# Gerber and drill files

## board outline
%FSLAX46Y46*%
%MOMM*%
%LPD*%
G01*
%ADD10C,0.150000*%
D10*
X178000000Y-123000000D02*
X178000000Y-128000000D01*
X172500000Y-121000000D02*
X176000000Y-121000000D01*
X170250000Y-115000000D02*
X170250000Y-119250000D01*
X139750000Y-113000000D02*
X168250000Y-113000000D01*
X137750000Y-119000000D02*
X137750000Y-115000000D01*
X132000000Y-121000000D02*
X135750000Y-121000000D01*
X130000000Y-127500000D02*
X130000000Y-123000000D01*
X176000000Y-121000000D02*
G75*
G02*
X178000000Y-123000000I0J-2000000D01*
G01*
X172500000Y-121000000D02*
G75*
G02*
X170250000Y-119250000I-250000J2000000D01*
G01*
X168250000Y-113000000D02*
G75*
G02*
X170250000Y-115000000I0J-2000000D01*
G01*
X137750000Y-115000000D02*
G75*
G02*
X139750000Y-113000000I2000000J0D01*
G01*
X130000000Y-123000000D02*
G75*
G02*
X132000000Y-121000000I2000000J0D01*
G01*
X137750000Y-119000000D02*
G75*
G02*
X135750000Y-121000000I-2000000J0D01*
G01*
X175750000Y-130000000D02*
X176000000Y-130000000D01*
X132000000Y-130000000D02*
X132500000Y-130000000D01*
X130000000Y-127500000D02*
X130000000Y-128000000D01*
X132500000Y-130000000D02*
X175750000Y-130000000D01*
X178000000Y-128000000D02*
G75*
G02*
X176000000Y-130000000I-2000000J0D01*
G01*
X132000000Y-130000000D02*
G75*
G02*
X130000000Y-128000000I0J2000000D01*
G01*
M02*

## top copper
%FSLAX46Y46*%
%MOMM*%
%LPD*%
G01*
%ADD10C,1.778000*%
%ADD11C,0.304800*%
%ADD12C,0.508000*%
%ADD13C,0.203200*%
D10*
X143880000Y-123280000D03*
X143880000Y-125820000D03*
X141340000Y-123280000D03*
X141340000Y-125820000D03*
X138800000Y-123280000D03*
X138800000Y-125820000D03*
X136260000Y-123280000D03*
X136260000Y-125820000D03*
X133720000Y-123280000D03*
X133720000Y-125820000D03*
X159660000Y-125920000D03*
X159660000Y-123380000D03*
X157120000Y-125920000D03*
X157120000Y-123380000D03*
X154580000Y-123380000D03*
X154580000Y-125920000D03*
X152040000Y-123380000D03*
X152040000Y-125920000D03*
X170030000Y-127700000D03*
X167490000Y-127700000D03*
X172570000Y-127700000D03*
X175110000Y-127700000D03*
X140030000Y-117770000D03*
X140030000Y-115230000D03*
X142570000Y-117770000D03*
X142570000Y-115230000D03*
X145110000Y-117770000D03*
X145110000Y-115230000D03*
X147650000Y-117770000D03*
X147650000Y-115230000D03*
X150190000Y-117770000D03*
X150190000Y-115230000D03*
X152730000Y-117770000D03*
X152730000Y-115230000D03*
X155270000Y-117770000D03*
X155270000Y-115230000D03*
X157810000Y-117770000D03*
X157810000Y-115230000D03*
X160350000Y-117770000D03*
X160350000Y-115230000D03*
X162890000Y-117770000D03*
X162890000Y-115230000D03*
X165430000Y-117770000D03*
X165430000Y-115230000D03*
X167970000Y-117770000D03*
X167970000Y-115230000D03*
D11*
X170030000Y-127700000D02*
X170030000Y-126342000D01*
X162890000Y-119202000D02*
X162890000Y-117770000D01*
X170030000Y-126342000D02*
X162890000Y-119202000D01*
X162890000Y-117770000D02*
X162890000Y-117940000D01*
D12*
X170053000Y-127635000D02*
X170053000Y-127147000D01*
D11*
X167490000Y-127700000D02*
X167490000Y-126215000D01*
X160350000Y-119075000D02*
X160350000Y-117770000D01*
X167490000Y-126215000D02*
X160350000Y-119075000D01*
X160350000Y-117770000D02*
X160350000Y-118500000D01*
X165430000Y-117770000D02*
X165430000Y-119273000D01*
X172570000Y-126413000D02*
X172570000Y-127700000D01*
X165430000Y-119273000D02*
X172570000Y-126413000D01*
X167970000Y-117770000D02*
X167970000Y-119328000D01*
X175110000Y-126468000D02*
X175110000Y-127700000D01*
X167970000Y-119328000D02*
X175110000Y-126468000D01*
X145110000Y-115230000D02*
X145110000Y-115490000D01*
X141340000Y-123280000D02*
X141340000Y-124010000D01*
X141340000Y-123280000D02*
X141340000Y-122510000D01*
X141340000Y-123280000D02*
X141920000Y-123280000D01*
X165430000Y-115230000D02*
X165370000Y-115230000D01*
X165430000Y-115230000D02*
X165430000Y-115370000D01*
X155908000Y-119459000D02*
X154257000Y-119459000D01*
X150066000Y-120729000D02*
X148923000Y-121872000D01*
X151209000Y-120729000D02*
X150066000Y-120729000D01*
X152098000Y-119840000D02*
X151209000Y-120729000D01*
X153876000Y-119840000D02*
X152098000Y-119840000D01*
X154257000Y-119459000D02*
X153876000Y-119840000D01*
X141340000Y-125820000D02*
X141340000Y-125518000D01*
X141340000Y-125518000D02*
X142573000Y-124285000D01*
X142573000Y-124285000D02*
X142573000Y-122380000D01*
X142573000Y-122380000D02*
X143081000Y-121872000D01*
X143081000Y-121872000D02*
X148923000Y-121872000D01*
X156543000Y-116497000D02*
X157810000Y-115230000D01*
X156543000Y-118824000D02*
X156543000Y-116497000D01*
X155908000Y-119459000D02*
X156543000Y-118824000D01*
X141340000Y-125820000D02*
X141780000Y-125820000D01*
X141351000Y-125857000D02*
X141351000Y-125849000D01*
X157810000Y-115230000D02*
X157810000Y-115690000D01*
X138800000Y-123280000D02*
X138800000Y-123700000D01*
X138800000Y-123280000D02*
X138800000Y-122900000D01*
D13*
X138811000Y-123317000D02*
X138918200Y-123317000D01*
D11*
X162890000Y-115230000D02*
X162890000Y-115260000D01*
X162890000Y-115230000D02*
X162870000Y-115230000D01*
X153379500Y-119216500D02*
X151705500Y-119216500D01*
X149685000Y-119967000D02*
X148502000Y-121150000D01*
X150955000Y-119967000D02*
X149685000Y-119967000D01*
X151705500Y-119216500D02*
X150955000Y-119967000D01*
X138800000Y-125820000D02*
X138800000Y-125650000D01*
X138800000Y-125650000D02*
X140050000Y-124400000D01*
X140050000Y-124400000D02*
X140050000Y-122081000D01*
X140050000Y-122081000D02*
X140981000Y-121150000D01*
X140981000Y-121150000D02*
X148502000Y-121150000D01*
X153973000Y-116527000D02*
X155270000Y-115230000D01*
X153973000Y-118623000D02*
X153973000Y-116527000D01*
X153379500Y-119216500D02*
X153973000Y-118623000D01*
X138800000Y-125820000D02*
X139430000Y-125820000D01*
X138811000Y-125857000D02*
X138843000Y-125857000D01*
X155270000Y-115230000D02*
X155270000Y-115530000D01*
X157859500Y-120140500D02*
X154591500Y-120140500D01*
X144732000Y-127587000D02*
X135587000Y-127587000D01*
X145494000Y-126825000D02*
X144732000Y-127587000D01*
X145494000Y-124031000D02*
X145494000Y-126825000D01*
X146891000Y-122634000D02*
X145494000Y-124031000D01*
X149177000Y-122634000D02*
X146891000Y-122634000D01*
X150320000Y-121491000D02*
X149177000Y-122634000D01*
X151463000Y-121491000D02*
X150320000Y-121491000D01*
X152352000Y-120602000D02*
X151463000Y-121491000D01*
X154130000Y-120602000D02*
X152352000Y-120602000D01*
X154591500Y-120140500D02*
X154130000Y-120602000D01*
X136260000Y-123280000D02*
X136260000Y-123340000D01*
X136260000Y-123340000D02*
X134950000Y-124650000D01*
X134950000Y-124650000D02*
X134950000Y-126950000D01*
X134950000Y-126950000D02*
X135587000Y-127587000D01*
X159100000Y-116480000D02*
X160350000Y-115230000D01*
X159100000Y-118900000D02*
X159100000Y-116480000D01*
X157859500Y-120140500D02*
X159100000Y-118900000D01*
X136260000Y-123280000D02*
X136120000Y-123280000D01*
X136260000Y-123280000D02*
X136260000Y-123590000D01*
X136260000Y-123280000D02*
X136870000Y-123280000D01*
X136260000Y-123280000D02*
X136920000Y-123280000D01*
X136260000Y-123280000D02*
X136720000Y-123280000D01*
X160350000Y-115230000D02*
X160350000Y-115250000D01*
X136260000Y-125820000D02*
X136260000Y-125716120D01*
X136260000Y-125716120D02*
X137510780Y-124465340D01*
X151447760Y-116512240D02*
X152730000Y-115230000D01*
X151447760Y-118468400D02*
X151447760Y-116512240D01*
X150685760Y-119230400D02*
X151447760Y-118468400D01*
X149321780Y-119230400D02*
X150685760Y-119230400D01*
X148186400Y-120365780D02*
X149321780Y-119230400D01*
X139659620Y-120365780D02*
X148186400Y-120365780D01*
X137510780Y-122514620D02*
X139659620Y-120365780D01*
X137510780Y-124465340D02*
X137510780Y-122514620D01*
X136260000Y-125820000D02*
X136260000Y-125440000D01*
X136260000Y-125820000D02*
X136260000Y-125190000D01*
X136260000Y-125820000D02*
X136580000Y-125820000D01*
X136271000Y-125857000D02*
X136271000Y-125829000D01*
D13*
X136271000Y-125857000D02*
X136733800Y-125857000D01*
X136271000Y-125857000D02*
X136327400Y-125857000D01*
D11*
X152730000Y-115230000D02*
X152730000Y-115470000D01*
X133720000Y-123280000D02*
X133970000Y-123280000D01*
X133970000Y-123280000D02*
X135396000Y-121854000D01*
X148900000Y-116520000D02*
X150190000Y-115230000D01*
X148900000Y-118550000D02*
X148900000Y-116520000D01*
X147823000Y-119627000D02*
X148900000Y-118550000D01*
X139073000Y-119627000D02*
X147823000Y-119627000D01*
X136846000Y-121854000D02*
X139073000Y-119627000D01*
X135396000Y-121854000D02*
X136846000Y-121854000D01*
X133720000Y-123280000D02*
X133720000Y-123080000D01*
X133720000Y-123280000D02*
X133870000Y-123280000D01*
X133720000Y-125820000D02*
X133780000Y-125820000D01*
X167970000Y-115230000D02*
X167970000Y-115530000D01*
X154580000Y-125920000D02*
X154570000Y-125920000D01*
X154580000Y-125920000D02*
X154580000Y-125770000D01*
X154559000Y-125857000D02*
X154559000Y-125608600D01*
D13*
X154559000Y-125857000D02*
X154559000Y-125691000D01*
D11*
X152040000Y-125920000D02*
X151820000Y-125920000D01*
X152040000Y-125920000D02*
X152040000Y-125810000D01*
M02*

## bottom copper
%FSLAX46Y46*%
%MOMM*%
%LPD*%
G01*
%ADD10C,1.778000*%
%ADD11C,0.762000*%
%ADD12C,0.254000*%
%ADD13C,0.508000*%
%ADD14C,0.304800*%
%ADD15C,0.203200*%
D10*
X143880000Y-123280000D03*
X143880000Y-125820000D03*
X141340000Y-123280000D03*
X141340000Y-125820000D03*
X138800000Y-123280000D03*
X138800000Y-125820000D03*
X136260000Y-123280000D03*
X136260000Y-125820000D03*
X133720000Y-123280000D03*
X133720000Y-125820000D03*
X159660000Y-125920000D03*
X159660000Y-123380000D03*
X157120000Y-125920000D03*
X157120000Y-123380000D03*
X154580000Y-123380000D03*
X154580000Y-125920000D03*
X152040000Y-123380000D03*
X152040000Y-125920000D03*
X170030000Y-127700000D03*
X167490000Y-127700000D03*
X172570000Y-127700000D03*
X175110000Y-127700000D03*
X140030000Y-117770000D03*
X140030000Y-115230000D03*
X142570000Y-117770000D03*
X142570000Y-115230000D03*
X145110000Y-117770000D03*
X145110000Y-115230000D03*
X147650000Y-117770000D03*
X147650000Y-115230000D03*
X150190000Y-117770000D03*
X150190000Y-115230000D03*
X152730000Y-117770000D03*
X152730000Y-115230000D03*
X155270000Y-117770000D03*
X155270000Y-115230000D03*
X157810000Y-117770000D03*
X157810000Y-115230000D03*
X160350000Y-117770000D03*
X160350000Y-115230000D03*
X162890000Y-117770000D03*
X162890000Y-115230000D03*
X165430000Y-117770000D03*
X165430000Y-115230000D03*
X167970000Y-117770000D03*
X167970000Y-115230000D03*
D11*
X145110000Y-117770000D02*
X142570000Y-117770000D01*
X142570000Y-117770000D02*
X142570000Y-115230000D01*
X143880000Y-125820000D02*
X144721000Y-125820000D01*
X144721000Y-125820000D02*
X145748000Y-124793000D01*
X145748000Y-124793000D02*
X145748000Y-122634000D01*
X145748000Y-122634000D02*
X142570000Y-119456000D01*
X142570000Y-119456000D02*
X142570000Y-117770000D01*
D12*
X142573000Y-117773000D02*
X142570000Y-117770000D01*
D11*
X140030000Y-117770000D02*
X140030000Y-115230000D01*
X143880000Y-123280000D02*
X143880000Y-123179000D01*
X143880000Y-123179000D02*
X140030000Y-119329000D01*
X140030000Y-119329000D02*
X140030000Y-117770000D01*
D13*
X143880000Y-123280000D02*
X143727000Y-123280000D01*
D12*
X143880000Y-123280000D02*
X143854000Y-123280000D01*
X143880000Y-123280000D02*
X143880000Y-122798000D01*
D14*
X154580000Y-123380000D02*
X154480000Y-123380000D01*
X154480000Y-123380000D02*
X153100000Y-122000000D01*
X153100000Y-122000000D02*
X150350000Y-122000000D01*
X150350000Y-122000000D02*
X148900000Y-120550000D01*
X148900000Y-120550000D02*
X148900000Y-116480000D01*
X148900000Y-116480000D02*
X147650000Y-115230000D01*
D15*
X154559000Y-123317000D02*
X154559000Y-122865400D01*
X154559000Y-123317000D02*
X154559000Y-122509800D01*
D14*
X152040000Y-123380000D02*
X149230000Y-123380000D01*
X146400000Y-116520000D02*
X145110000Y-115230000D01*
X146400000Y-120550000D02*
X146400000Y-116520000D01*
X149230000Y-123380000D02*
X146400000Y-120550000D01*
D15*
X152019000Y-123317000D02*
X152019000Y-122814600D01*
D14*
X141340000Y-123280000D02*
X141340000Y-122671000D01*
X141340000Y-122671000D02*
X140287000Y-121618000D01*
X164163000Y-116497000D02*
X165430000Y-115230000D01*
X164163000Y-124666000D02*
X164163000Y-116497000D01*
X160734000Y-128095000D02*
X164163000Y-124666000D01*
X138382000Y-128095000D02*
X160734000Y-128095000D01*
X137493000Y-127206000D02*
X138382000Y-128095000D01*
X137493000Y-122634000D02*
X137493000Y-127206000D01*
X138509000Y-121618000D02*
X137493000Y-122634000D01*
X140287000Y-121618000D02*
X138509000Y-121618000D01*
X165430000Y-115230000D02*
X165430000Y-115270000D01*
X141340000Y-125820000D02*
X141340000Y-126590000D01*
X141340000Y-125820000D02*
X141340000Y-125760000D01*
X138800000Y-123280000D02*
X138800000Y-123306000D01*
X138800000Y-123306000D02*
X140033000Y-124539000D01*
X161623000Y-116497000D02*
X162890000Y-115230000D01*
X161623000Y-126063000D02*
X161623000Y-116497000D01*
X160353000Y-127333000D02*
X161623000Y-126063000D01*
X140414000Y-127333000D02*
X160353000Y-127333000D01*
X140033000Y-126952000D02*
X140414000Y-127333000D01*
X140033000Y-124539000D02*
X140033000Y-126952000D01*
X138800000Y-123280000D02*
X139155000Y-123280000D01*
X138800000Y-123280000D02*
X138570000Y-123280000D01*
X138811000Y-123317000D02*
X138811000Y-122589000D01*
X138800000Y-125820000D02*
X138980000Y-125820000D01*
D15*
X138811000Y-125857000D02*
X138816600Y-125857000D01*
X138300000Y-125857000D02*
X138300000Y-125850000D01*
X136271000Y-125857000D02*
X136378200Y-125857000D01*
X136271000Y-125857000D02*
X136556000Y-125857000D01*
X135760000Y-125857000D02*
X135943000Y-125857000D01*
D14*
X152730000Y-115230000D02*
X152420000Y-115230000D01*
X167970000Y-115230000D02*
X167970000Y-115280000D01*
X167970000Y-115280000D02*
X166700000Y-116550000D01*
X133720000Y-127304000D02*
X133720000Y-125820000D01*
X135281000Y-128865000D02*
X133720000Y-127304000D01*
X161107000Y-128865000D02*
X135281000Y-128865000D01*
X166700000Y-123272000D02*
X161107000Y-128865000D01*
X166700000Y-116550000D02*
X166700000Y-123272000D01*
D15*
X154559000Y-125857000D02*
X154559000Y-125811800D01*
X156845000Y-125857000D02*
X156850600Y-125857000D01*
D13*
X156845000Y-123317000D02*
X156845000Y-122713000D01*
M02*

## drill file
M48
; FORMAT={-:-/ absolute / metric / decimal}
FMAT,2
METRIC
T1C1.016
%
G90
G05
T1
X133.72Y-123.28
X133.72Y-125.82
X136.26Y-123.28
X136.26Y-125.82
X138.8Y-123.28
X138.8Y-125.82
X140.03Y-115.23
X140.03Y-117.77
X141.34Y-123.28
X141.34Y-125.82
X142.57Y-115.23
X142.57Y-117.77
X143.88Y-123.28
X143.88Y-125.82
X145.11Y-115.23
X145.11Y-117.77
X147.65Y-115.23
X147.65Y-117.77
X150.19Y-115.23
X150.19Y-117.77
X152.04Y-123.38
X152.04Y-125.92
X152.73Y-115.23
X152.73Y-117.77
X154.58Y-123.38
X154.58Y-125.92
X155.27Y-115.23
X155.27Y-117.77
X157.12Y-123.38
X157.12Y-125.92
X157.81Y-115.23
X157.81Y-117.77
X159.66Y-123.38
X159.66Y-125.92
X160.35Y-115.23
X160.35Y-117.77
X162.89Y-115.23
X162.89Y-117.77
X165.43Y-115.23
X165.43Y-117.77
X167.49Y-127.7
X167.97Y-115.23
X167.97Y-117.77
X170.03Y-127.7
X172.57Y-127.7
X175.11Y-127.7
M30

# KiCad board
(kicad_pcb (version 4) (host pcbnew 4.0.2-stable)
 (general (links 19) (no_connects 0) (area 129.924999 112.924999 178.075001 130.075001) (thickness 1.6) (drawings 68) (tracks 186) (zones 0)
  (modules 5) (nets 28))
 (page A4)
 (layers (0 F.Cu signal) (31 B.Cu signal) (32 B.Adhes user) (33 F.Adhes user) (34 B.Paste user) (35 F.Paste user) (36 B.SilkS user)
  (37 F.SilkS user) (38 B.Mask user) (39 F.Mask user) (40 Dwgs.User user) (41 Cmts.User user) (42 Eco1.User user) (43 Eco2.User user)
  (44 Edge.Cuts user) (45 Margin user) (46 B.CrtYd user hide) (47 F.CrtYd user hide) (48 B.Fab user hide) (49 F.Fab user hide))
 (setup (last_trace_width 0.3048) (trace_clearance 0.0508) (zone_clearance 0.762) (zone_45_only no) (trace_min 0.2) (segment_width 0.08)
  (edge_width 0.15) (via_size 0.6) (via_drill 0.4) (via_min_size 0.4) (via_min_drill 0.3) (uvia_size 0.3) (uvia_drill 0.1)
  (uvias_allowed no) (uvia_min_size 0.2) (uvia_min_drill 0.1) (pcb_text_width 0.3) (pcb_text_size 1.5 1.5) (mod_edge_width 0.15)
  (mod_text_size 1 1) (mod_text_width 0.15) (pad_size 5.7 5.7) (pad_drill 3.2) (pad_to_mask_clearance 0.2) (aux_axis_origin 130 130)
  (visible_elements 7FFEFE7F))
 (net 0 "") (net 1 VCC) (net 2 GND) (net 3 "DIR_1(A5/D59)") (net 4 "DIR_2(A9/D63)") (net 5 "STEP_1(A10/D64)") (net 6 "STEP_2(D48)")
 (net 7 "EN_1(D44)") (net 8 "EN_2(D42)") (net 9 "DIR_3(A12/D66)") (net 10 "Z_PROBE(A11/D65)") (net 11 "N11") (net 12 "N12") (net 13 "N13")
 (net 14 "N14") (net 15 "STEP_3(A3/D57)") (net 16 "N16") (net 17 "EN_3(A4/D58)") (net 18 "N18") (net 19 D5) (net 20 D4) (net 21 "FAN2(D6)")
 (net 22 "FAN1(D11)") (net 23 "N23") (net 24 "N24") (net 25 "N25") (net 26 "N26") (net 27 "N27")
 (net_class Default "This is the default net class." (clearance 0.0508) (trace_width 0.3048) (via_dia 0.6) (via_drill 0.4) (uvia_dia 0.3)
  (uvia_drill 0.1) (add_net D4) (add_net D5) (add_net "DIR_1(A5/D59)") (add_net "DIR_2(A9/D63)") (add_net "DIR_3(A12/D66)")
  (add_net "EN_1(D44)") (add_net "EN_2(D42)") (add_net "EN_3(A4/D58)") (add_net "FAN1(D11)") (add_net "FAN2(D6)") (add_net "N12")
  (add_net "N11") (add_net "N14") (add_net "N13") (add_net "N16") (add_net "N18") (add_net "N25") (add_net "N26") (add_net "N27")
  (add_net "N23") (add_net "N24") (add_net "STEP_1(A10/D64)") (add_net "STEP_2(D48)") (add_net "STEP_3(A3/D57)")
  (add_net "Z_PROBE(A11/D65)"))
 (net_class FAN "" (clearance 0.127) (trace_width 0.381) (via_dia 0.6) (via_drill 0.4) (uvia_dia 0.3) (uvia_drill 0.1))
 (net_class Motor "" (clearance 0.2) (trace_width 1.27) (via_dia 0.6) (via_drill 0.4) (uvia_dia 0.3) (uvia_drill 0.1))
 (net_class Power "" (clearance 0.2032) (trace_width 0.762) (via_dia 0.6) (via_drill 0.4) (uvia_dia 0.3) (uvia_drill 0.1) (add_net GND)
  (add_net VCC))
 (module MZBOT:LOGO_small (layer F.Cu) (at 167.66058 124.78538)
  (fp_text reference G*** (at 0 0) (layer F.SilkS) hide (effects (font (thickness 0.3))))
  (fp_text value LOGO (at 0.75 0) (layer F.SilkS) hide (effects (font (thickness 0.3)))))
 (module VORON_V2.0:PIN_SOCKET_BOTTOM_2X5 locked (layer F.Cu) (at 138.8 124.55 180)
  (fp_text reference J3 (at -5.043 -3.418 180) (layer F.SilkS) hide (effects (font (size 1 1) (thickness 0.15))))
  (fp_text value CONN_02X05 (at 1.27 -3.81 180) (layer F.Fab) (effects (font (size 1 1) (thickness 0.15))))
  (pad 1 thru_hole circle (at -5.08 1.27 180) (size 1.778 1.778) (drill 1.016) (layers *.Cu *.Mask F.SilkS) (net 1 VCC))
  (pad 2 thru_hole circle (at -5.08 -1.27 180) (size 1.778 1.778) (drill 1.016) (layers *.Cu *.Mask F.SilkS) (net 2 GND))
  (pad 3 thru_hole circle (at -2.54 1.27 180) (size 1.778 1.778) (drill 1.016) (layers *.Cu *.Mask F.SilkS) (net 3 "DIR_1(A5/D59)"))
  (pad 4 thru_hole circle (at -2.54 -1.27 180) (size 1.778 1.778) (drill 1.016) (layers *.Cu *.Mask F.SilkS) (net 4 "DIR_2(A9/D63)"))
  (pad 5 thru_hole circle (at 0 1.27 180) (size 1.778 1.778) (drill 1.016) (layers *.Cu *.Mask F.SilkS) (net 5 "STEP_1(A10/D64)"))
  (pad 6 thru_hole circle (at 0 -1.27 180) (size 1.778 1.778) (drill 1.016) (layers *.Cu *.Mask F.SilkS) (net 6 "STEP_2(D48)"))
  (pad 7 thru_hole circle (at 2.54 1.27 180) (size 1.778 1.778) (drill 1.016) (layers *.Cu *.Mask F.SilkS) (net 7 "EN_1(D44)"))
  (pad 8 thru_hole circle (at 2.54 -1.27 180) (size 1.778 1.778) (drill 1.016) (layers *.Cu *.Mask F.SilkS) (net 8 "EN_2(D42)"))
  (pad 9 thru_hole circle (at 5.08 1.27 180) (size 1.778 1.778) (drill 1.016) (layers *.Cu *.Mask F.SilkS) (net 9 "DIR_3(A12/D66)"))
  (pad 10 thru_hole circle (at 5.08 -1.27 180) (size 1.778 1.778) (drill 1.016) (layers *.Cu *.Mask F.SilkS) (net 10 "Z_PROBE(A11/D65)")))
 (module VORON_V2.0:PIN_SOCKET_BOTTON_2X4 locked (layer F.Cu) (at 155.85 124.65 180)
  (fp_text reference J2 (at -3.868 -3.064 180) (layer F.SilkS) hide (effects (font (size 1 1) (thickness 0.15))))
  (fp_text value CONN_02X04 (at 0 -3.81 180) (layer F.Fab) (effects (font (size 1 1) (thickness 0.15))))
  (pad 2 thru_hole circle (at -3.81 -1.27 180) (size 1.778 1.778) (drill 1.016) (layers *.Cu *.Mask F.SilkS) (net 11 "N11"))
  (pad 1 thru_hole circle (at -3.81 1.27 180) (size 1.778 1.778) (drill 1.016) (layers *.Cu *.Mask F.SilkS) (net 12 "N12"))
  (pad 4 thru_hole circle (at -1.27 -1.27 180) (size 1.778 1.778) (drill 1.016) (layers *.Cu *.Mask F.SilkS) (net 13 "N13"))
  (pad 3 thru_hole circle (at -1.27 1.27 180) (size 1.778 1.778) (drill 1.016) (layers *.Cu *.Mask F.SilkS) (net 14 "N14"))
  (pad 5 thru_hole circle (at 1.27 1.27 180) (size 1.778 1.778) (drill 1.016) (layers *.Cu *.Mask F.SilkS) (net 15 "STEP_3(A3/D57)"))
  (pad 6 thru_hole circle (at 1.27 -1.27 180) (size 1.778 1.778) (drill 1.016) (layers *.Cu *.Mask F.SilkS) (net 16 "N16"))
  (pad 7 thru_hole circle (at 3.81 1.27 180) (size 1.778 1.778) (drill 1.016) (layers *.Cu *.Mask F.SilkS) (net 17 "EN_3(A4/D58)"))
  (pad 8 thru_hole circle (at 3.81 -1.27 180) (size 1.778 1.778) (drill 1.016) (layers *.Cu *.Mask F.SilkS) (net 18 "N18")))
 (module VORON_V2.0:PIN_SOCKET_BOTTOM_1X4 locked (layer F.Cu) (at 171.3 127.7)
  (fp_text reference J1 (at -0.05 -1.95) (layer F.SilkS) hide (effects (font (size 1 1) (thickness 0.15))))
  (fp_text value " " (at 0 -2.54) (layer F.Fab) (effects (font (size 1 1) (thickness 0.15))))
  (pad 2 thru_hole circle (at -1.27 0) (size 1.778 1.778) (drill 1.016) (layers *.Cu *.Mask F.SilkS) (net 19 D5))
  (pad 1 thru_hole circle (at -3.81 0) (size 1.778 1.778) (drill 1.016) (layers *.Cu *.Mask F.SilkS) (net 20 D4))
  (pad 3 thru_hole circle (at 1.27 0) (size 1.778 1.778) (drill 1.016) (layers *.Cu *.Mask F.SilkS) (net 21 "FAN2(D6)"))
  (pad 4 thru_hole circle (at 3.81 0) (size 1.778 1.778) (drill 1.016) (layers *.Cu *.Mask F.SilkS) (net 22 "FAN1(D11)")))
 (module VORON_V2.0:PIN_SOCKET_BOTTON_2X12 (layer F.Cu) (at 154 116.5)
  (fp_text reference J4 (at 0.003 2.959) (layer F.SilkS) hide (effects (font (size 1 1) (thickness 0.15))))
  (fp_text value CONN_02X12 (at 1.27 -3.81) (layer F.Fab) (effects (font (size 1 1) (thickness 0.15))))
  (pad 1 thru_hole circle (at -13.97 1.27) (size 1.778 1.778) (drill 1.016) (layers *.Cu *.Mask F.SilkS) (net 1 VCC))
  (pad 2 thru_hole circle (at -13.97 -1.27) (size 1.778 1.778) (drill 1.016) (layers *.Cu *.Mask F.SilkS) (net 1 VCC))
  (pad 3 thru_hole circle (at -11.43 1.27) (size 1.778 1.778) (drill 1.016) (layers *.Cu *.Mask F.SilkS) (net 2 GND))
  (pad 4 thru_hole circle (at -11.43 -1.27) (size 1.778 1.778) (drill 1.016) (layers *.Cu *.Mask F.SilkS) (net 2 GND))
  (pad 5 thru_hole circle (at -8.89 1.27) (size 1.778 1.778) (drill 1.016) (layers *.Cu *.Mask F.SilkS) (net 2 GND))
  (pad 6 thru_hole circle (at -8.89 -1.27) (size 1.778 1.778) (drill 1.016) (layers *.Cu *.Mask F.SilkS) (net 17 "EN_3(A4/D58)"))
  (pad 7 thru_hole circle (at -6.35 1.27) (size 1.778 1.778) (drill 1.016) (layers *.Cu *.Mask F.SilkS) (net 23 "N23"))
  (pad 8 thru_hole circle (at -6.35 -1.27) (size 1.778 1.778) (drill 1.016) (layers *.Cu *.Mask F.SilkS) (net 15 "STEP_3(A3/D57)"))
  (pad 9 thru_hole circle (at -3.81 1.27) (size 1.778 1.778) (drill 1.016) (layers *.Cu *.Mask F.SilkS) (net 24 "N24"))
  (pad 10 thru_hole circle (at -3.81 -1.27) (size 1.778 1.778) (drill 1.016) (layers *.Cu *.Mask F.SilkS) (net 9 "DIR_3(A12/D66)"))
  (pad 11 thru_hole circle (at -1.27 1.27) (size 1.778 1.778) (drill 1.016) (layers *.Cu *.Mask F.SilkS) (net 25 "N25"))
  (pad 12 thru_hole circle (at -1.27 -1.27) (size 1.778 1.778) (drill 1.016) (layers *.Cu *.Mask F.SilkS) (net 8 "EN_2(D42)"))
  (pad 13 thru_hole circle (at 1.27 1.27) (size 1.778 1.778) (drill 1.016) (layers *.Cu *.Mask F.SilkS) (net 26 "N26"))
  (pad 14 thru_hole circle (at 1.27 -1.27) (size 1.778 1.778) (drill 1.016) (layers *.Cu *.Mask F.SilkS) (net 6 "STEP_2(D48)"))
  (pad 15 thru_hole circle (at 3.81 1.27) (size 1.778 1.778) (drill 1.016) (layers *.Cu *.Mask F.SilkS) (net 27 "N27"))
  (pad 16 thru_hole circle (at 3.81 -1.27) (size 1.778 1.778) (drill 1.016) (layers *.Cu *.Mask F.SilkS) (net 4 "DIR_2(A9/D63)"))
  (pad 17 thru_hole circle (at 6.35 1.27) (size 1.778 1.778) (drill 1.016) (layers *.Cu *.Mask F.SilkS) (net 20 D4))
  (pad 18 thru_hole circle (at 6.35 -1.27) (size 1.778 1.778) (drill 1.016) (layers *.Cu *.Mask F.SilkS) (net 7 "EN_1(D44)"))
  (pad 19 thru_hole circle (at 8.89 1.27) (size 1.778 1.778) (drill 1.016) (layers *.Cu *.Mask F.SilkS) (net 19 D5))
  (pad 20 thru_hole circle (at 8.89 -1.27) (size 1.778 1.778) (drill 1.016) (layers *.Cu *.Mask F.SilkS) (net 5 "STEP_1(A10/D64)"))
  (pad 21 thru_hole circle (at 11.43 1.27) (size 1.778 1.778) (drill 1.016) (layers *.Cu *.Mask F.SilkS) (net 21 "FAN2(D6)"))
  (pad 22 thru_hole circle (at 11.43 -1.27) (size 1.778 1.778) (drill 1.016) (layers *.Cu *.Mask F.SilkS) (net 3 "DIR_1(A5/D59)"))
  (pad 23 thru_hole circle (at 13.97 1.27) (size 1.778 1.778) (drill 1.016) (layers *.Cu *.Mask F.SilkS) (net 22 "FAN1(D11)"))
  (pad 24 thru_hole circle (at 13.97 -1.27) (size 1.778 1.778) (drill 1.016) (layers *.Cu *.Mask F.SilkS) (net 10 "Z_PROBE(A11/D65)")))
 (gr_line (start 178 123) (end 178 128) (angle 90) (layer Edge.Cuts) (width 0.15))
 (gr_line (start 172.5 121) (end 176 121) (angle 90) (layer Edge.Cuts) (width 0.15))
 (gr_line (start 170.25 115) (end 170.25 119.25) (angle 90) (layer Edge.Cuts) (width 0.15))
 (gr_line (start 139.75 113) (end 168.25 113) (angle 90) (layer Edge.Cuts) (width 0.15))
 (gr_line (start 137.75 119) (end 137.75 115) (angle 90) (layer Edge.Cuts) (width 0.15))
 (gr_line (start 132 121) (end 135.75 121) (angle 90) (layer Edge.Cuts) (width 0.15))
 (gr_line (start 130 127.5) (end 130 123) (angle 90) (layer Edge.Cuts) (width 0.15))
 (gr_arc (start 176 123) (end 176 121) (angle 90) (layer Edge.Cuts) (width 0.15))
 (gr_arc (start 172.25 119) (end 172.5 121) (angle 90) (layer Edge.Cuts) (width 0.15))
 (gr_arc (start 168.25 115) (end 168.25 113) (angle 90) (layer Edge.Cuts) (width 0.15))
 (gr_arc (start 139.75 115) (end 137.75 115) (angle 90) (layer Edge.Cuts) (width 0.15))
 (gr_arc (start 132 123) (end 130 123) (angle 90) (layer Edge.Cuts) (width 0.15))
 (gr_arc (start 135.75 119) (end 137.75 119) (angle 90) (layer Edge.Cuts) (width 0.15))
 (gr_line (start 175.75 130) (end 176 130) (angle 90) (layer Edge.Cuts) (width 0.15))
 (gr_line (start 132 130) (end 132.5 130) (angle 90) (layer Edge.Cuts) (width 0.15))
 (gr_line (start 130 127.5) (end 130 128) (angle 90) (layer Edge.Cuts) (width 0.15))
 (gr_line (start 132.5 130) (end 175.75 130) (angle 90) (layer Edge.Cuts) (width 0.15))
 (gr_arc (start 176 128) (end 178 128) (angle 90) (layer Edge.Cuts) (width 0.15))
 (gr_arc (start 132 128) (end 132 130) (angle 90) (layer Edge.Cuts) (width 0.15))
 (segment (start 145.11 117.77) (end 142.57 117.77) (width 0.762) (layer B.Cu) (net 2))
 (segment (start 142.57 117.77) (end 142.57 115.23) (width 0.762) (layer B.Cu) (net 2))
 (segment (start 143.88 125.82) (end 144.721 125.82) (width 0.762) (layer B.Cu) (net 2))
 (segment (start 144.721 125.82) (end 145.748 124.793) (width 0.762) (layer B.Cu) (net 2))
 (segment (start 145.748 124.793) (end 145.748 122.634) (width 0.762) (layer B.Cu) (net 2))
 (segment (start 145.748 122.634) (end 142.57 119.456) (width 0.762) (layer B.Cu) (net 2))
 (segment (start 142.57 119.456) (end 142.57 117.77) (width 0.762) (layer B.Cu) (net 2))
 (segment (start 142.573 117.773) (end 142.57 117.77) (width 0.254) (layer B.Cu) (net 2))
 (segment (start 140.03 117.77) (end 140.03 115.23) (width 0.762) (layer B.Cu) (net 1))
 (segment (start 143.88 123.28) (end 143.88 123.179) (width 0.762) (layer B.Cu) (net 1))
 (segment (start 143.88 123.179) (end 140.03 119.329) (width 0.762) (layer B.Cu) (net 1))
 (segment (start 140.03 119.329) (end 140.03 117.77) (width 0.762) (layer B.Cu) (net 1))
 (segment (start 143.88 123.28) (end 143.727 123.28) (width 0.508) (layer B.Cu) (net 1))
 (segment (start 143.88 123.28) (end 143.854 123.28) (width 0.254) (layer B.Cu) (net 1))
 (segment (start 143.88 123.28) (end 143.88 122.798) (width 0.254) (layer B.Cu) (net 1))
 (segment (start 170.03 127.7) (end 170.03 126.342) (width 0.3048) (layer F.Cu) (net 19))
 (segment (start 162.89 119.202) (end 162.89 117.77) (width 0.3048) (layer F.Cu) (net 19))
 (segment (start 170.03 126.342) (end 162.89 119.202) (width 0.3048) (layer F.Cu) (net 19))
 (segment (start 162.89 117.77) (end 162.89 117.94) (width 0.3048) (layer F.Cu) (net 19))
 (segment (start 170.053 127.635) (end 170.053 127.147) (width 0.508) (layer F.Cu) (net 19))
 (segment (start 167.49 127.7) (end 167.49 126.215) (width 0.3048) (layer F.Cu) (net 20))
 (segment (start 160.35 119.075) (end 160.35 117.77) (width 0.3048) (layer F.Cu) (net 20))
 (segment (start 167.49 126.215) (end 160.35 119.075) (width 0.3048) (layer F.Cu) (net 20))
 (segment (start 160.35 117.77) (end 160.35 118.5) (width 0.3048) (layer F.Cu) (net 20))
 (segment (start 165.43 117.77) (end 165.43 119.273) (width 0.3048) (layer F.Cu) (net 21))
 (segment (start 172.57 126.413) (end 172.57 127.7) (width 0.3048) (layer F.Cu) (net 21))
 (segment (start 165.43 119.273) (end 172.57 126.413) (width 0.3048) (layer F.Cu) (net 21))
 (segment (start 167.97 117.77) (end 167.97 119.328) (width 0.3048) (layer F.Cu) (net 22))
 (segment (start 175.11 126.468) (end 175.11 127.7) (width 0.3048) (layer F.Cu) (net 22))
 (segment (start 167.97 119.328) (end 175.11 126.468) (width 0.3048) (layer F.Cu) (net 22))
 (segment (start 154.58 123.38) (end 154.48 123.38) (width 0.3048) (layer B.Cu) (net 15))
 (segment (start 154.48 123.38) (end 153.1 122) (width 0.3048) (layer B.Cu) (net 15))
 (segment (start 153.1 122) (end 150.35 122) (width 0.3048) (layer B.Cu) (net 15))
 (segment (start 150.35 122) (end 148.9 120.55) (width 0.3048) (layer B.Cu) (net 15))
 (segment (start 148.9 120.55) (end 148.9 116.48) (width 0.3048) (layer B.Cu) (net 15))
 (segment (start 148.9 116.48) (end 147.65 115.23) (width 0.3048) (layer B.Cu) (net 15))
 (segment (start 154.559 123.317) (end 154.559 122.8654) (width 0.2032) (layer B.Cu) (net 15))
 (segment (start 154.559 123.317) (end 154.559 122.5098) (width 0.2032) (layer B.Cu) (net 15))
 (segment (start 152.04 123.38) (end 149.23 123.38) (width 0.3048) (layer B.Cu) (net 17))
 (segment (start 146.4 116.52) (end 145.11 115.23) (width 0.3048) (layer B.Cu) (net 17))
 (segment (start 146.4 120.55) (end 146.4 116.52) (width 0.3048) (layer B.Cu) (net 17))
 (segment (start 149.23 123.38) (end 146.4 120.55) (width 0.3048) (layer B.Cu) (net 17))
 (segment (start 152.019 123.317) (end 152.019 122.8146) (width 0.2032) (layer B.Cu) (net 17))
 (segment (start 145.11 115.23) (end 145.11 115.49) (width 0.3048) (layer F.Cu) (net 17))
 (segment (start 141.34 123.28) (end 141.34 122.671) (width 0.3048) (layer B.Cu) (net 3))
 (segment (start 141.34 122.671) (end 140.287 121.618) (width 0.3048) (layer B.Cu) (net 3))
 (segment (start 164.163 116.497) (end 165.43 115.23) (width 0.3048) (layer B.Cu) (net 3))
 (segment (start 164.163 124.666) (end 164.163 116.497) (width 0.3048) (layer B.Cu) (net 3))
 (segment (start 160.734 128.095) (end 164.163 124.666) (width 0.3048) (layer B.Cu) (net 3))
 (segment (start 138.382 128.095) (end 160.734 128.095) (width 0.3048) (layer B.Cu) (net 3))
 (segment (start 137.493 127.206) (end 138.382 128.095) (width 0.3048) (layer B.Cu) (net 3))
 (segment (start 137.493 122.634) (end 137.493 127.206) (width 0.3048) (layer B.Cu) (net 3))
 (segment (start 138.509 121.618) (end 137.493 122.634) (width 0.3048) (layer B.Cu) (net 3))
 (segment (start 140.287 121.618) (end 138.509 121.618) (width 0.3048) (layer B.Cu) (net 3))
 (segment (start 165.43 115.23) (end 165.43 115.27) (width 0.3048) (layer B.Cu) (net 3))
 (segment (start 141.34 123.28) (end 141.34 124.01) (width 0.3048) (layer F.Cu) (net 3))
 (segment (start 141.34 123.28) (end 141.34 122.51) (width 0.3048) (layer F.Cu) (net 3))
 (segment (start 141.34 123.28) (end 141.92 123.28) (width 0.3048) (layer F.Cu) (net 3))
 (segment (start 165.43 115.23) (end 165.37 115.23) (width 0.3048) (layer F.Cu) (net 3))
 (segment (start 165.43 115.23) (end 165.43 115.37) (width 0.3048) (layer F.Cu) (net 3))
 (segment (start 155.908 119.459) (end 154.257 119.459) (width 0.3048) (layer F.Cu) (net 4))
 (segment (start 150.066 120.729) (end 148.923 121.872) (width 0.3048) (layer F.Cu) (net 4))
 (segment (start 151.209 120.729) (end 150.066 120.729) (width 0.3048) (layer F.Cu) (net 4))
 (segment (start 152.098 119.84) (end 151.209 120.729) (width 0.3048) (layer F.Cu) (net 4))
 (segment (start 153.876 119.84) (end 152.098 119.84) (width 0.3048) (layer F.Cu) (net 4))
 (segment (start 154.257 119.459) (end 153.876 119.84) (width 0.3048) (layer F.Cu) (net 4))
 (segment (start 141.34 125.82) (end 141.34 125.518) (width 0.3048) (layer F.Cu) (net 4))
 (segment (start 141.34 125.518) (end 142.573 124.285) (width 0.3048) (layer F.Cu) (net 4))
 (segment (start 142.573 124.285) (end 142.573 122.38) (width 0.3048) (layer F.Cu) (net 4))
 (segment (start 142.573 122.38) (end 143.081 121.872) (width 0.3048) (layer F.Cu) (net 4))
 (segment (start 143.081 121.872) (end 148.923 121.872) (width 0.3048) (layer F.Cu) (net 4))
 (segment (start 156.543 116.497) (end 157.81 115.23) (width 0.3048) (layer F.Cu) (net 4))
 (segment (start 156.543 118.824) (end 156.543 116.497) (width 0.3048) (layer F.Cu) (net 4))
 (segment (start 155.908 119.459) (end 156.543 118.824) (width 0.3048) (layer F.Cu) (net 4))
 (segment (start 141.34 125.82) (end 141.34 126.59) (width 0.3048) (layer B.Cu) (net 4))
 (segment (start 141.34 125.82) (end 141.34 125.76) (width 0.3048) (layer B.Cu) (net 4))
 (segment (start 141.34 125.82) (end 141.78 125.82) (width 0.3048) (layer F.Cu) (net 4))
 (segment (start 141.351 125.857) (end 141.351 125.849) (width 0.3048) (layer F.Cu) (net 4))
 (segment (start 157.81 115.23) (end 157.81 115.69) (width 0.3048) (layer F.Cu) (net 4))
 (segment (start 138.8 123.28) (end 138.8 123.306) (width 0.3048) (layer B.Cu) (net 5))
 (segment (start 138.8 123.306) (end 140.033 124.539) (width 0.3048) (layer B.Cu) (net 5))
 (segment (start 161.623 116.497) (end 162.89 115.23) (width 0.3048) (layer B.Cu) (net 5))
 (segment (start 161.623 126.063) (end 161.623 116.497) (width 0.3048) (layer B.Cu) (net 5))
 (segment (start 160.353 127.333) (end 161.623 126.063) (width 0.3048) (layer B.Cu) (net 5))
 (segment (start 140.414 127.333) (end 160.353 127.333) (width 0.3048) (layer B.Cu) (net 5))
 (segment (start 140.033 126.952) (end 140.414 127.333) (width 0.3048) (layer B.Cu) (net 5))
 (segment (start 140.033 124.539) (end 140.033 126.952) (width 0.3048) (layer B.Cu) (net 5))
 (segment (start 138.8 123.28) (end 139.155 123.28) (width 0.3048) (layer B.Cu) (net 5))
 (segment (start 138.8 123.28) (end 138.57 123.28) (width 0.3048) (layer B.Cu) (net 5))
 (segment (start 138.8 123.28) (end 138.8 123.7) (width 0.3048) (layer F.Cu) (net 5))
 (segment (start 138.8 123.28) (end 138.8 122.9) (width 0.3048) (layer F.Cu) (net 5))
 (segment (start 138.811 123.317) (end 138.9182 123.317) (width 0.2032) (layer F.Cu) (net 5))
 (segment (start 138.811 123.317) (end 138.811 122.589) (width 0.3048) (layer B.Cu) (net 5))
 (segment (start 162.89 115.23) (end 162.89 115.26) (width 0.3048) (layer F.Cu) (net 5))
 (segment (start 162.89 115.23) (end 162.87 115.23) (width 0.3048) (layer F.Cu) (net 5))
 (segment (start 153.3795 119.2165) (end 151.7055 119.2165) (width 0.3048) (layer F.Cu) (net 6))
 (segment (start 149.685 119.967) (end 148.502 121.15) (width 0.3048) (layer F.Cu) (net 6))
 (segment (start 150.955 119.967) (end 149.685 119.967) (width 0.3048) (layer F.Cu) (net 6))
 (segment (start 151.7055 119.2165) (end 150.955 119.967) (width 0.3048) (layer F.Cu) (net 6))
 (segment (start 138.8 125.82) (end 138.8 125.65) (width 0.3048) (layer F.Cu) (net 6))
 (segment (start 138.8 125.65) (end 140.05 124.4) (width 0.3048) (layer F.Cu) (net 6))
 (segment (start 140.05 124.4) (end 140.05 122.081) (width 0.3048) (layer F.Cu) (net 6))
 (segment (start 140.05 122.081) (end 140.981 121.15) (width 0.3048) (layer F.Cu) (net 6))
 (segment (start 140.981 121.15) (end 148.502 121.15) (width 0.3048) (layer F.Cu) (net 6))
 (segment (start 153.973 116.527) (end 155.27 115.23) (width 0.3048) (layer F.Cu) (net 6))
 (segment (start 153.973 118.623) (end 153.973 116.527) (width 0.3048) (layer F.Cu) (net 6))
 (segment (start 153.3795 119.2165) (end 153.973 118.623) (width 0.3048) (layer F.Cu) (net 6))
 (segment (start 138.8 125.82) (end 139.43 125.82) (width 0.3048) (layer F.Cu) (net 6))
 (segment (start 138.8 125.82) (end 138.98 125.82) (width 0.3048) (layer B.Cu) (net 6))
 (segment (start 138.811 125.857) (end 138.8166 125.857) (width 0.2032) (layer B.Cu) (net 6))
 (segment (start 138.3 125.857) (end 138.3 125.85) (width 0.2032) (layer B.Cu) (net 6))
 (segment (start 138.811 125.857) (end 138.843 125.857) (width 0.3048) (layer F.Cu) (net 6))
 (segment (start 155.27 115.23) (end 155.27 115.53) (width 0.3048) (layer F.Cu) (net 6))
 (segment (start 157.8595 120.1405) (end 154.5915 120.1405) (width 0.3048) (layer F.Cu) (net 7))
 (segment (start 144.732 127.587) (end 135.587 127.587) (width 0.3048) (layer F.Cu) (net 7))
 (segment (start 145.494 126.825) (end 144.732 127.587) (width 0.3048) (layer F.Cu) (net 7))
 (segment (start 145.494 124.031) (end 145.494 126.825) (width 0.3048) (layer F.Cu) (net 7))
 (segment (start 146.891 122.634) (end 145.494 124.031) (width 0.3048) (layer F.Cu) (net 7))
 (segment (start 149.177 122.634) (end 146.891 122.634) (width 0.3048) (layer F.Cu) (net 7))
 (segment (start 150.32 121.491) (end 149.177 122.634) (width 0.3048) (layer F.Cu) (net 7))
 (segment (start 151.463 121.491) (end 150.32 121.491) (width 0.3048) (layer F.Cu) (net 7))
 (segment (start 152.352 120.602) (end 151.463 121.491) (width 0.3048) (layer F.Cu) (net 7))
 (segment (start 154.13 120.602) (end 152.352 120.602) (width 0.3048) (layer F.Cu) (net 7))
 (segment (start 154.5915 120.1405) (end 154.13 120.602) (width 0.3048) (layer F.Cu) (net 7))
 (segment (start 136.26 123.28) (end 136.26 123.34) (width 0.3048) (layer F.Cu) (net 7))
 (segment (start 136.26 123.34) (end 134.95 124.65) (width 0.3048) (layer F.Cu) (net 7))
 (segment (start 134.95 124.65) (end 134.95 126.95) (width 0.3048) (layer F.Cu) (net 7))
 (segment (start 134.95 126.95) (end 135.587 127.587) (width 0.3048) (layer F.Cu) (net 7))
 (segment (start 159.1 116.48) (end 160.35 115.23) (width 0.3048) (layer F.Cu) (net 7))
 (segment (start 159.1 118.9) (end 159.1 116.48) (width 0.3048) (layer F.Cu) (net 7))
 (segment (start 157.8595 120.1405) (end 159.1 118.9) (width 0.3048) (layer F.Cu) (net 7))
 (segment (start 136.26 123.28) (end 136.12 123.28) (width 0.3048) (layer F.Cu) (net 7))
 (segment (start 136.26 123.28) (end 136.26 123.59) (width 0.3048) (layer F.Cu) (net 7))
 (segment (start 136.26 123.28) (end 136.87 123.28) (width 0.3048) (layer F.Cu) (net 7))
 (segment (start 136.26 123.28) (end 136.92 123.28) (width 0.3048) (layer F.Cu) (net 7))
 (segment (start 136.26 123.28) (end 136.72 123.28) (width 0.3048) (layer F.Cu) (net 7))
 (segment (start 160.35 115.23) (end 160.35 115.25) (width 0.3048) (layer F.Cu) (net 7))
 (segment (start 136.26 125.82) (end 136.26 125.71612) (width 0.3048) (layer F.Cu) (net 8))
 (segment (start 136.26 125.71612) (end 137.51078 124.46534) (width 0.3048) (layer F.Cu) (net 8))
 (segment (start 151.44776 116.51224) (end 152.73 115.23) (width 0.3048) (layer F.Cu) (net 8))
 (segment (start 151.44776 118.4684) (end 151.44776 116.51224) (width 0.3048) (layer F.Cu) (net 8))
 (segment (start 150.68576 119.2304) (end 151.44776 118.4684) (width 0.3048) (layer F.Cu) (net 8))
 (segment (start 149.32178 119.2304) (end 150.68576 119.2304) (width 0.3048) (layer F.Cu) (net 8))
 (segment (start 148.1864 120.36578) (end 149.32178 119.2304) (width 0.3048) (layer F.Cu) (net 8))
 (segment (start 139.65962 120.36578) (end 148.1864 120.36578) (width 0.3048) (layer F.Cu) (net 8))
 (segment (start 137.51078 122.51462) (end 139.65962 120.36578) (width 0.3048) (layer F.Cu) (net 8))
 (segment (start 137.51078 124.46534) (end 137.51078 122.51462) (width 0.3048) (layer F.Cu) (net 8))
 (segment (start 136.26 125.82) (end 136.26 125.44) (width 0.3048) (layer F.Cu) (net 8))
 (segment (start 136.26 125.82) (end 136.26 125.19) (width 0.3048) (layer F.Cu) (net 8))
 (segment (start 136.26 125.82) (end 136.58 125.82) (width 0.3048) (layer F.Cu) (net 8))
 (segment (start 136.271 125.857) (end 136.3782 125.857) (width 0.2032) (layer B.Cu) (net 8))
 (segment (start 136.271 125.857) (end 136.556 125.857) (width 0.2032) (layer B.Cu) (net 8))
 (segment (start 135.76 125.857) (end 135.943 125.857) (width 0.2032) (layer B.Cu) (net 8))
 (segment (start 136.271 125.857) (end 136.271 125.829) (width 0.3048) (layer F.Cu) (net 8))
 (segment (start 136.271 125.857) (end 136.7338 125.857) (width 0.2032) (layer F.Cu) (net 8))
 (segment (start 136.271 125.857) (end 136.3274 125.857) (width 0.2032) (layer F.Cu) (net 8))
 (segment (start 152.73 115.23) (end 152.42 115.23) (width 0.3048) (layer B.Cu) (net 8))
 (segment (start 152.73 115.23) (end 152.73 115.47) (width 0.3048) (layer F.Cu) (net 8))
 (segment (start 133.72 123.28) (end 133.97 123.28) (width 0.3048) (layer F.Cu) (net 9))
 (segment (start 133.97 123.28) (end 135.396 121.854) (width 0.3048) (layer F.Cu) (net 9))
 (segment (start 148.9 116.52) (end 150.19 115.23) (width 0.3048) (layer F.Cu) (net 9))
 (segment (start 148.9 118.55) (end 148.9 116.52) (width 0.3048) (layer F.Cu) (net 9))
 (segment (start 147.823 119.627) (end 148.9 118.55) (width 0.3048) (layer F.Cu) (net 9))
 (segment (start 139.073 119.627) (end 147.823 119.627) (width 0.3048) (layer F.Cu) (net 9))
 (segment (start 136.846 121.854) (end 139.073 119.627) (width 0.3048) (layer F.Cu) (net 9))
 (segment (start 135.396 121.854) (end 136.846 121.854) (width 0.3048) (layer F.Cu) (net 9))
 (segment (start 133.72 123.28) (end 133.72 123.08) (width 0.3048) (layer F.Cu) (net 9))
 (segment (start 133.72 123.28) (end 133.87 123.28) (width 0.3048) (layer F.Cu) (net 9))
 (segment (start 167.97 115.23) (end 167.97 115.28) (width 0.3048) (layer B.Cu) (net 10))
 (segment (start 167.97 115.28) (end 166.7 116.55) (width 0.3048) (layer B.Cu) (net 10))
 (segment (start 133.72 127.304) (end 133.72 125.82) (width 0.3048) (layer B.Cu) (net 10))
 (segment (start 135.281 128.865) (end 133.72 127.304) (width 0.3048) (layer B.Cu) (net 10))
 (segment (start 161.107 128.865) (end 135.281 128.865) (width 0.3048) (layer B.Cu) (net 10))
 (segment (start 166.7 123.272) (end 161.107 128.865) (width 0.3048) (layer B.Cu) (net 10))
 (segment (start 166.7 116.55) (end 166.7 123.272) (width 0.3048) (layer B.Cu) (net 10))
 (segment (start 133.72 125.82) (end 133.78 125.82) (width 0.3048) (layer F.Cu) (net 10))
 (segment (start 167.97 115.23) (end 167.97 115.53) (width 0.3048) (layer F.Cu) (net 10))
 (segment (start 154.58 125.92) (end 154.57 125.92) (width 0.3048) (layer F.Cu) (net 16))
 (segment (start 154.58 125.92) (end 154.58 125.77) (width 0.3048) (layer F.Cu) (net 16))
 (segment (start 154.559 125.857) (end 154.559 125.8118) (width 0.2032) (layer B.Cu) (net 16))
 (segment (start 154.559 125.857) (end 154.559 125.6086) (width 0.3048) (layer F.Cu) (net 16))
 (segment (start 154.559 125.857) (end 154.559 125.691) (width 0.2032) (layer F.Cu) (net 16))
 (segment (start 152.04 125.92) (end 151.82 125.92) (width 0.3048) (layer F.Cu) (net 18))
 (segment (start 152.04 125.92) (end 152.04 125.81) (width 0.3048) (layer F.Cu) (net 18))
 (segment (start 156.845 125.857) (end 156.8506 125.857) (width 0.2032) (layer B.Cu) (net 13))
 (segment (start 156.845 123.317) (end 156.845 122.713) (width 0.508) (layer B.Cu) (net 14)))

